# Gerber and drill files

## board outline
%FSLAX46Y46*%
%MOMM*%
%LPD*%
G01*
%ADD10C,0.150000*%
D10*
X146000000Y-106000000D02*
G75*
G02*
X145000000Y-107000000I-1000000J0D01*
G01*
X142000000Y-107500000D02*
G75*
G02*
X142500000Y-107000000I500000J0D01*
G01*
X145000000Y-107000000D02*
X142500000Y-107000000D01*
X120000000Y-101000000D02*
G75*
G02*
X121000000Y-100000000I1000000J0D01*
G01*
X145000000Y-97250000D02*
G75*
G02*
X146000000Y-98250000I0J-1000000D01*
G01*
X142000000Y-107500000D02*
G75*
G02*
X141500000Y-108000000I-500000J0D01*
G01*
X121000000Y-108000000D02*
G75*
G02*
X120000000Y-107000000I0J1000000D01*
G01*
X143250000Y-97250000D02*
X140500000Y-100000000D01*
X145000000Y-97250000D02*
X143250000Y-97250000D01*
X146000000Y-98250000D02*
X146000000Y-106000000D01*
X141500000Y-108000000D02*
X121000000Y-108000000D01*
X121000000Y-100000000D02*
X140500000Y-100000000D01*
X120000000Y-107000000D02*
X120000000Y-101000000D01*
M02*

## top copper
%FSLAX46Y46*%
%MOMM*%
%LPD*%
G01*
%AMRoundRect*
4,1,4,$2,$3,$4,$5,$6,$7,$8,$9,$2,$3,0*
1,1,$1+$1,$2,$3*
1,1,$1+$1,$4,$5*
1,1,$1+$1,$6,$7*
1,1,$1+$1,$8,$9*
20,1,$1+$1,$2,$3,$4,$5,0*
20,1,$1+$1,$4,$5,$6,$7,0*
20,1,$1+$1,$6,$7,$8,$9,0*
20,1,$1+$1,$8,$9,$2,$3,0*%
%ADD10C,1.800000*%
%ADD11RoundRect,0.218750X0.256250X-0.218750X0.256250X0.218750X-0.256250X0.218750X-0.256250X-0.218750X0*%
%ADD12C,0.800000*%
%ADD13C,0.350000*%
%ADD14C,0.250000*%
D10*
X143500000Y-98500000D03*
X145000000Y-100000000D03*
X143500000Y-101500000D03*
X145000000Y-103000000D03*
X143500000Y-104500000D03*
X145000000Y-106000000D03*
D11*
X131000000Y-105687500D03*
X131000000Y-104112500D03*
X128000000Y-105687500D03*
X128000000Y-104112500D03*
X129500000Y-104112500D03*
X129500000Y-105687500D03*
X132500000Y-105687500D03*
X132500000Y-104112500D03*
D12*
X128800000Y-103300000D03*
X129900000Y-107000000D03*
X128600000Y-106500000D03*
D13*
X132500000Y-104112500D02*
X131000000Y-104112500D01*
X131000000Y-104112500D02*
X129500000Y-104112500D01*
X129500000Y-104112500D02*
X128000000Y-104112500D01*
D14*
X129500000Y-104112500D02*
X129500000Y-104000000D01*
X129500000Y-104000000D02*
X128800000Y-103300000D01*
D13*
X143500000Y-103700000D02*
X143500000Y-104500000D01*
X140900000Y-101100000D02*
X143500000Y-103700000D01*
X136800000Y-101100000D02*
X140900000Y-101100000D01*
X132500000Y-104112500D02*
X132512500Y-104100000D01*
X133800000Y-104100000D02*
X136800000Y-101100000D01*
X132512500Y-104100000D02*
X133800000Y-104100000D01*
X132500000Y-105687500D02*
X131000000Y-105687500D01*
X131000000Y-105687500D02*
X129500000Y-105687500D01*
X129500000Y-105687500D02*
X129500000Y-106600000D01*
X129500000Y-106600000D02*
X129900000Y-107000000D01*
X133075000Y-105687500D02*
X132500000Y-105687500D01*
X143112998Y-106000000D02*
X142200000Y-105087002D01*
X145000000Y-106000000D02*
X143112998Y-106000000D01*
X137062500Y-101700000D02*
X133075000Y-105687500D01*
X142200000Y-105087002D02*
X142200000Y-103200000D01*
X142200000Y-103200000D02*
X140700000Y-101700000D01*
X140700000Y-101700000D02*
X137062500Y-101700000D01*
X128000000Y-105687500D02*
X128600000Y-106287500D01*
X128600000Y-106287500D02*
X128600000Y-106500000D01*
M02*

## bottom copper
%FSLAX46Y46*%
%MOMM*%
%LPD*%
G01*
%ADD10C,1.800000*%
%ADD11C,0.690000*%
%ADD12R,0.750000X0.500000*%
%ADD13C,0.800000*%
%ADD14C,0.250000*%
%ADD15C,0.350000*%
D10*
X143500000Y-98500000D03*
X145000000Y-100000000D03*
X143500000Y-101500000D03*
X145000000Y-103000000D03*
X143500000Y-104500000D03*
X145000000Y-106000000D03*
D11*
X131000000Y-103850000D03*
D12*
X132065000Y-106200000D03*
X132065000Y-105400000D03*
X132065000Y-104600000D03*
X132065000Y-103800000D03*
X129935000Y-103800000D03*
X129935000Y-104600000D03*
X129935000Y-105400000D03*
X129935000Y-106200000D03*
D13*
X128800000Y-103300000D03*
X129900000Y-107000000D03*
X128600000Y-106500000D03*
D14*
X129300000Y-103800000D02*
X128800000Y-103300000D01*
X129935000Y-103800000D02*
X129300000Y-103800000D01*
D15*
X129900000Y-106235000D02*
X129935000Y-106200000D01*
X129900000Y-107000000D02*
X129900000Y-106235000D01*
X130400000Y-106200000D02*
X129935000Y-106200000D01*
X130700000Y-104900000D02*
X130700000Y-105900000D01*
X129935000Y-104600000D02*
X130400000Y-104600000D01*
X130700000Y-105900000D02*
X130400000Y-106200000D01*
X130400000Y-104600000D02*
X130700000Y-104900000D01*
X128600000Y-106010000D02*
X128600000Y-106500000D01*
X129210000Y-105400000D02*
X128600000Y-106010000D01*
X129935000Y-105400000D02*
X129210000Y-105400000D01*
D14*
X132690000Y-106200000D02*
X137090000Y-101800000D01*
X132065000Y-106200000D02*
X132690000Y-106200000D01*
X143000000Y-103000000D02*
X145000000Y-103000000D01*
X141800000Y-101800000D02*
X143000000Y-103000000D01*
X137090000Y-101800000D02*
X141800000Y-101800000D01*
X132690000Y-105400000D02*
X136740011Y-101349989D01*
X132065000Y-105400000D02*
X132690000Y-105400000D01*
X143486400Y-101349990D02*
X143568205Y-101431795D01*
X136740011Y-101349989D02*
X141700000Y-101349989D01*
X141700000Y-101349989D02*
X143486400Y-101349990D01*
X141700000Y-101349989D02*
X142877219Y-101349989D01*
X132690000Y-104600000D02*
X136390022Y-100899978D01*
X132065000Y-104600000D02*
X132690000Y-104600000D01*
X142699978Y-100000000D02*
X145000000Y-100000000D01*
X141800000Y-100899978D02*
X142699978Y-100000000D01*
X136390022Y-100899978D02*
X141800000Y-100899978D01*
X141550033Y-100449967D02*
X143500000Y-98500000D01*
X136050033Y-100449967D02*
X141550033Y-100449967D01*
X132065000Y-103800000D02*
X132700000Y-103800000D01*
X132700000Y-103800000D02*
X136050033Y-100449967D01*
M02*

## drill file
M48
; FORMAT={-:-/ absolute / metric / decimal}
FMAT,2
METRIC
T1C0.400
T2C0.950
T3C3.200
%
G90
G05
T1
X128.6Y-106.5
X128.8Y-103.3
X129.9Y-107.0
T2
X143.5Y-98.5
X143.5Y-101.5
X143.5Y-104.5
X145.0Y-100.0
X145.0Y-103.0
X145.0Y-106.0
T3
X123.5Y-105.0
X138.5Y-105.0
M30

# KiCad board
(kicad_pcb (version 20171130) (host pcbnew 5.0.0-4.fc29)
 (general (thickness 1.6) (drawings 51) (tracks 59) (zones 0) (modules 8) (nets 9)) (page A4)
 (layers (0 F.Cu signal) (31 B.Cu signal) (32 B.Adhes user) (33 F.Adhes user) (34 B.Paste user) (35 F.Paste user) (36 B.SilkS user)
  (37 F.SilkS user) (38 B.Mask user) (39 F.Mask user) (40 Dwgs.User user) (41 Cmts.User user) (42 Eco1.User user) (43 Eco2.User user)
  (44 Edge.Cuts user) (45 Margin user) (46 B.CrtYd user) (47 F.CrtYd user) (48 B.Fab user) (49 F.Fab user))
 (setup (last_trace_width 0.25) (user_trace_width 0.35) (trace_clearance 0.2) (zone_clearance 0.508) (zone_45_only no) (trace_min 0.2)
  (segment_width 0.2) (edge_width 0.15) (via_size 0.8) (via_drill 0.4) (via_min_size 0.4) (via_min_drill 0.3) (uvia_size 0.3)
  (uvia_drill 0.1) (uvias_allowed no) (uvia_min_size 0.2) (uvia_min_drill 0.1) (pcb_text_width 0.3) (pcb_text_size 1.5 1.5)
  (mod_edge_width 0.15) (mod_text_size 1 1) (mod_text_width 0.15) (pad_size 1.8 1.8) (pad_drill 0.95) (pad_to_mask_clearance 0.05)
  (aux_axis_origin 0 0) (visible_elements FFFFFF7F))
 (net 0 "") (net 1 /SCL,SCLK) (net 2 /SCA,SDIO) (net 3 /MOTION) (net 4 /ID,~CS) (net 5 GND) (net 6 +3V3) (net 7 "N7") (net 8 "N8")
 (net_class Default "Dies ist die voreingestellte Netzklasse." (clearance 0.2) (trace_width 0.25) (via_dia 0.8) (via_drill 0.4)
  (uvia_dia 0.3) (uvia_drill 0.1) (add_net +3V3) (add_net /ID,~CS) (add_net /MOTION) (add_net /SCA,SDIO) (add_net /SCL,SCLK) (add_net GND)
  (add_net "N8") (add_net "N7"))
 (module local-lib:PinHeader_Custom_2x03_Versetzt (layer F.Cu) (at 145 106 180)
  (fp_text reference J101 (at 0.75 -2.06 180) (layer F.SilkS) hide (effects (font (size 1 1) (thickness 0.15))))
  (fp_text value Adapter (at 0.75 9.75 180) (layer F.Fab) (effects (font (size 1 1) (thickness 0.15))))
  (pad 6 thru_hole circle (at 1.5 7.5 180) (size 1.8 1.8) (drill 0.95) (layers *.Cu *.Mask) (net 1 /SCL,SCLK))
  (pad 5 thru_hole circle (at 0 6 180) (size 1.8 1.8) (drill 0.95) (layers *.Cu *.Mask) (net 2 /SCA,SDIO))
  (pad 4 thru_hole circle (at 1.5 4.5 180) (size 1.8 1.8) (drill 0.95) (layers *.Cu *.Mask) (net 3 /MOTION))
  (pad 3 thru_hole circle (at 0 3 180) (size 1.8 1.8) (drill 0.95) (layers *.Cu *.Mask) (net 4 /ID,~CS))
  (pad 2 thru_hole circle (at 1.5 1.5 180) (size 1.8 1.8) (drill 0.95) (layers *.Cu *.Mask) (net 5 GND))
  (pad 1 thru_hole circle (at 0 0 180) (size 1.8 1.8) (drill 0.95) (layers *.Cu *.Mask) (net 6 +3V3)))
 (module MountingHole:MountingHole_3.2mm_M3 (layer F.Cu) (at 138.5 105)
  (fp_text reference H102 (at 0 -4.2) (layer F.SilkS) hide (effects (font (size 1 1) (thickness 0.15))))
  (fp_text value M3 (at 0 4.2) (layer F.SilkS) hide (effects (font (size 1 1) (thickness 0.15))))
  (pad 1 np_thru_hole circle (at 0 0) (size 3.2 3.2) (drill 3.2) (layers *.Cu *.Mask)))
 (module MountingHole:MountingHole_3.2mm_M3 (layer F.Cu) (at 123.5 105)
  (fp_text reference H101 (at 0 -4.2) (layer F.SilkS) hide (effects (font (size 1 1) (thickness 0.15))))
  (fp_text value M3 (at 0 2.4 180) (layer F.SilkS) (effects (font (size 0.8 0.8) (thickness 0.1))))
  (pad 1 np_thru_hole circle (at 0 0) (size 3.2 3.2) (drill 3.2) (layers *.Cu *.Mask)))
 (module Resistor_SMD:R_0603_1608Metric (layer F.Cu) (at 131 104.9 90)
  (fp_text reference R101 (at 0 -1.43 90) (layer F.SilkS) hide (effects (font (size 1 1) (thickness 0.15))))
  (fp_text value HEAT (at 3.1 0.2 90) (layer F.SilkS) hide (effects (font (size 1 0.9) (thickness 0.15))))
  (pad 1 smd roundrect (at -0.7875 0 90) (size 0.875 0.95) (layers F.Cu F.Paste F.Mask) (roundrect_rratio 0.25) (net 6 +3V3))
  (pad 2 smd roundrect (at 0.7875 0 90) (size 0.875 0.95) (layers F.Cu F.Paste F.Mask) (roundrect_rratio 0.25) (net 5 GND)))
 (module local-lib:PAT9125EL (layer B.Cu) (at 131 105 90)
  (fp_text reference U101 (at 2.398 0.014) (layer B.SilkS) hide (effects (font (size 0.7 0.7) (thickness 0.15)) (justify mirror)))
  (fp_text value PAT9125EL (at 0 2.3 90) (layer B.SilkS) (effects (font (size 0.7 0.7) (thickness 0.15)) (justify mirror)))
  (pad 9 smd circle (at 1.15 0 90) (size 0.69 0.69) (layers B.Cu B.Paste B.Mask) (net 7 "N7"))
  (pad 8 smd rect (at -1.2 1.065 90) (size 0.5 0.75) (layers B.Cu B.Paste B.Mask) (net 4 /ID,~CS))
  (pad 7 smd rect (at -0.4 1.065 90) (size 0.5 0.75) (layers B.Cu B.Paste B.Mask) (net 3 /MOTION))
  (pad 6 smd rect (at 0.4 1.065 90) (size 0.5 0.75) (layers B.Cu B.Paste B.Mask) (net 2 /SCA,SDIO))
  (pad 5 smd rect (at 1.2 1.065 90) (size 0.5 0.75) (layers B.Cu B.Paste B.Mask) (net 1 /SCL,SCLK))
  (pad 4 smd rect (at 1.2 -1.065 90) (size 0.5 0.75) (layers B.Cu B.Paste B.Mask) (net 5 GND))
  (pad 3 smd rect (at 0.4 -1.065 90) (size 0.5 0.75) (layers B.Cu B.Paste B.Mask) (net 6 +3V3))
  (pad 2 smd rect (at -0.4 -1.065 90) (size 0.5 0.75) (layers B.Cu B.Paste B.Mask) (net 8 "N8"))
  (pad 1 smd rect (at -1.2 -1.065 90) (size 0.5 0.75) (layers B.Cu B.Paste B.Mask) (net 6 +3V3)))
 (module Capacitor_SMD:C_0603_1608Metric (layer F.Cu) (at 128 104.9 90)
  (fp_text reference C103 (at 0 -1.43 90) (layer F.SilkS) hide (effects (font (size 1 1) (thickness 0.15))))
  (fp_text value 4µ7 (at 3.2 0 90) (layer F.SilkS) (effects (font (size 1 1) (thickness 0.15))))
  (pad 1 smd roundrect (at -0.7875 0 90) (size 0.875 0.95) (layers F.Cu F.Paste F.Mask) (roundrect_rratio 0.25) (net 8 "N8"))
  (pad 2 smd roundrect (at 0.7875 0 90) (size 0.875 0.95) (layers F.Cu F.Paste F.Mask) (roundrect_rratio 0.25) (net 5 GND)))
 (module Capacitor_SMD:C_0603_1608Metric (layer F.Cu) (at 129.5 104.9 90)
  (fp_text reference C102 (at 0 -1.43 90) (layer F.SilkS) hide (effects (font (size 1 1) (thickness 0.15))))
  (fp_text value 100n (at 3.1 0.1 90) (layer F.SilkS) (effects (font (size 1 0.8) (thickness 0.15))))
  (pad 2 smd roundrect (at 0.7875 0 90) (size 0.875 0.95) (layers F.Cu F.Paste F.Mask) (roundrect_rratio 0.25) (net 5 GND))
  (pad 1 smd roundrect (at -0.7875 0 90) (size 0.875 0.95) (layers F.Cu F.Paste F.Mask) (roundrect_rratio 0.25) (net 6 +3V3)))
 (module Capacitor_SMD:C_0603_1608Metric (layer F.Cu) (at 132.5 104.9 90)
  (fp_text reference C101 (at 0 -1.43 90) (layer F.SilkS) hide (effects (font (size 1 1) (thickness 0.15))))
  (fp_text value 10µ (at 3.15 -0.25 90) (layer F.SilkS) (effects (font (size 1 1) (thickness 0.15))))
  (pad 1 smd roundrect (at -0.7875 0 90) (size 0.875 0.95) (layers F.Cu F.Paste F.Mask) (roundrect_rratio 0.25) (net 6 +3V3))
  (pad 2 smd roundrect (at 0.7875 0 90) (size 0.875 0.95) (layers F.Cu F.Paste F.Mask) (roundrect_rratio 0.25) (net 5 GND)))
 (gr_arc (start 145 106) (end 145 107) (angle -90) (layer Edge.Cuts) (width 0.15))
 (gr_arc (start 142.5 107.5) (end 142.5 107) (angle -90) (layer Edge.Cuts) (width 0.15))
 (gr_line (start 145 107) (end 142.5 107) (layer Edge.Cuts) (width 0.15))
 (gr_arc (start 121 101) (end 121 100) (angle -90) (layer Edge.Cuts) (width 0.15))
 (gr_arc (start 145 98.25) (end 146 98.25) (angle -90) (layer Edge.Cuts) (width 0.15))
 (gr_arc (start 141.5 107.5) (end 141.5 108) (angle -90) (layer Edge.Cuts) (width 0.15))
 (gr_arc (start 121 107) (end 120 107) (angle -90) (layer Edge.Cuts) (width 0.15))
 (gr_line (start 143.25 97.25) (end 140.5 100) (layer Edge.Cuts) (width 0.15))
 (gr_line (start 145 97.25) (end 143.25 97.25) (layer Edge.Cuts) (width 0.15))
 (gr_line (start 146 98.25) (end 146 106) (layer Edge.Cuts) (width 0.15))
 (gr_line (start 141.5 108) (end 121 108) (layer Edge.Cuts) (width 0.15))
 (gr_line (start 121 100) (end 140.5 100) (layer Edge.Cuts) (width 0.15))
 (gr_line (start 120 107) (end 120 101) (layer Edge.Cuts) (width 0.15))
 (segment (start 132.5 104.1125) (end 131 104.1125) (width 0.35) (layer F.Cu) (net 5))
 (segment (start 131 104.1125) (end 129.5 104.1125) (width 0.35) (layer F.Cu) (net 5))
 (segment (start 129.5 104.1125) (end 128 104.1125) (width 0.35) (layer F.Cu) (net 5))
 (via (at 128.8 103.3) (size 0.8) (drill 0.4) (layers F.Cu B.Cu) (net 5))
 (segment (start 129.5 104.1125) (end 129.5 104) (width 0.25) (layer F.Cu) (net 5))
 (segment (start 129.5 104) (end 128.8 103.3) (width 0.25) (layer F.Cu) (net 5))
 (segment (start 129.3 103.8) (end 128.8 103.3) (width 0.25) (layer B.Cu) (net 5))
 (segment (start 129.935 103.8) (end 129.3 103.8) (width 0.25) (layer B.Cu) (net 5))
 (segment (start 143.5 103.7) (end 143.5 104.5) (width 0.35) (layer F.Cu) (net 5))
 (segment (start 140.9 101.1) (end 143.5 103.7) (width 0.35) (layer F.Cu) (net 5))
 (segment (start 136.8 101.1) (end 140.9 101.1) (width 0.35) (layer F.Cu) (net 5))
 (segment (start 132.5 104.1125) (end 132.5125 104.1) (width 0.35) (layer F.Cu) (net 5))
 (segment (start 133.8 104.1) (end 136.8 101.1) (width 0.35) (layer F.Cu) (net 5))
 (segment (start 132.5125 104.1) (end 133.8 104.1) (width 0.35) (layer F.Cu) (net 5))
 (segment (start 132.5 105.6875) (end 131 105.6875) (width 0.35) (layer F.Cu) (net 6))
 (segment (start 131 105.6875) (end 129.5 105.6875) (width 0.35) (layer F.Cu) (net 6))
 (via (at 129.9 107) (size 0.8) (drill 0.4) (layers F.Cu B.Cu) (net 6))
 (segment (start 129.5 105.6875) (end 129.5 106.6) (width 0.35) (layer F.Cu) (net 6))
 (segment (start 129.5 106.6) (end 129.9 107) (width 0.35) (layer F.Cu) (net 6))
 (segment (start 129.9 106.235) (end 129.935 106.2) (width 0.35) (layer B.Cu) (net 6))
 (segment (start 129.9 107) (end 129.9 106.235) (width 0.35) (layer B.Cu) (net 6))
 (segment (start 130.4 106.2) (end 129.935 106.2) (width 0.35) (layer B.Cu) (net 6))
 (segment (start 130.7 104.9) (end 130.7 105.9) (width 0.35) (layer B.Cu) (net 6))
 (segment (start 129.935 104.6) (end 130.4 104.6) (width 0.35) (layer B.Cu) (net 6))
 (segment (start 130.7 105.9) (end 130.4 106.2) (width 0.35) (layer B.Cu) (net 6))
 (segment (start 130.4 104.6) (end 130.7 104.9) (width 0.35) (layer B.Cu) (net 6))
 (segment (start 133.075 105.6875) (end 132.5 105.6875) (width 0.35) (layer F.Cu) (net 6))
 (segment (start 143.112998 106) (end 142.2 105.087002) (width 0.35) (layer F.Cu) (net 6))
 (segment (start 145 106) (end 143.112998 106) (width 0.35) (layer F.Cu) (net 6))
 (segment (start 137.0625 101.7) (end 133.075 105.6875) (width 0.35) (layer F.Cu) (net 6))
 (segment (start 142.2 105.087002) (end 142.2 103.2) (width 0.35) (layer F.Cu) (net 6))
 (segment (start 142.2 103.2) (end 140.7 101.7) (width 0.35) (layer F.Cu) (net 6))
 (segment (start 140.7 101.7) (end 137.0625 101.7) (width 0.35) (layer F.Cu) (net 6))
 (segment (start 128 105.6875) (end 128.6 106.2875) (width 0.35) (layer F.Cu) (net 8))
 (segment (start 128.6 106.2875) (end 128.6 106.5) (width 0.35) (layer F.Cu) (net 8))
 (segment (start 128.6 106.01) (end 128.6 106.5) (width 0.35) (layer B.Cu) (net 8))
 (segment (start 129.21 105.4) (end 128.6 106.01) (width 0.35) (layer B.Cu) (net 8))
 (via (at 128.6 106.5) (size 0.8) (drill 0.4) (layers F.Cu B.Cu) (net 8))
 (segment (start 129.935 105.4) (end 129.21 105.4) (width 0.35) (layer B.Cu) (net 8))
 (segment (start 132.69 106.2) (end 137.09 101.8) (width 0.25) (layer B.Cu) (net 4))
 (segment (start 132.065 106.2) (end 132.69 106.2) (width 0.25) (layer B.Cu) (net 4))
 (segment (start 143 103) (end 145 103) (width 0.25) (layer B.Cu) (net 4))
 (segment (start 141.8 101.8) (end 143 103) (width 0.25) (layer B.Cu) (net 4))
 (segment (start 137.09 101.8) (end 141.8 101.8) (width 0.25) (layer B.Cu) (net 4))
 (segment (start 132.69 105.4) (end 136.740011 101.349989) (width 0.25) (layer B.Cu) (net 3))
 (segment (start 132.065 105.4) (end 132.69 105.4) (width 0.25) (layer B.Cu) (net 3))
 (segment (start 143.4864 101.34999) (end 143.568205 101.431795) (width 0.25) (layer B.Cu) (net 3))
 (segment (start 136.740011 101.349989) (end 141.7 101.349989) (width 0.25) (layer B.Cu) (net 3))
 (segment (start 141.7 101.349989) (end 143.4864 101.34999) (width 0.25) (layer B.Cu) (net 3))
 (segment (start 141.7 101.349989) (end 142.877219 101.349989) (width 0.25) (layer B.Cu) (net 3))
 (segment (start 132.69 104.6) (end 136.390022 100.899978) (width 0.25) (layer B.Cu) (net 2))
 (segment (start 132.065 104.6) (end 132.69 104.6) (width 0.25) (layer B.Cu) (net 2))
 (segment (start 142.699978 100) (end 145 100) (width 0.25) (layer B.Cu) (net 2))
 (segment (start 141.8 100.899978) (end 142.699978 100) (width 0.25) (layer B.Cu) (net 2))
 (segment (start 136.390022 100.899978) (end 141.8 100.899978) (width 0.25) (layer B.Cu) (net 2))
 (segment (start 141.550033 100.449967) (end 143.5 98.5) (width 0.25) (layer B.Cu) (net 1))
 (segment (start 136.050033 100.449967) (end 141.550033 100.449967) (width 0.25) (layer B.Cu) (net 1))
 (segment (start 132.065 103.8) (end 132.7 103.8) (width 0.25) (layer B.Cu) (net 1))
 (segment (start 132.7 103.8) (end 136.050033 100.449967) (width 0.25) (layer B.Cu) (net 1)))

